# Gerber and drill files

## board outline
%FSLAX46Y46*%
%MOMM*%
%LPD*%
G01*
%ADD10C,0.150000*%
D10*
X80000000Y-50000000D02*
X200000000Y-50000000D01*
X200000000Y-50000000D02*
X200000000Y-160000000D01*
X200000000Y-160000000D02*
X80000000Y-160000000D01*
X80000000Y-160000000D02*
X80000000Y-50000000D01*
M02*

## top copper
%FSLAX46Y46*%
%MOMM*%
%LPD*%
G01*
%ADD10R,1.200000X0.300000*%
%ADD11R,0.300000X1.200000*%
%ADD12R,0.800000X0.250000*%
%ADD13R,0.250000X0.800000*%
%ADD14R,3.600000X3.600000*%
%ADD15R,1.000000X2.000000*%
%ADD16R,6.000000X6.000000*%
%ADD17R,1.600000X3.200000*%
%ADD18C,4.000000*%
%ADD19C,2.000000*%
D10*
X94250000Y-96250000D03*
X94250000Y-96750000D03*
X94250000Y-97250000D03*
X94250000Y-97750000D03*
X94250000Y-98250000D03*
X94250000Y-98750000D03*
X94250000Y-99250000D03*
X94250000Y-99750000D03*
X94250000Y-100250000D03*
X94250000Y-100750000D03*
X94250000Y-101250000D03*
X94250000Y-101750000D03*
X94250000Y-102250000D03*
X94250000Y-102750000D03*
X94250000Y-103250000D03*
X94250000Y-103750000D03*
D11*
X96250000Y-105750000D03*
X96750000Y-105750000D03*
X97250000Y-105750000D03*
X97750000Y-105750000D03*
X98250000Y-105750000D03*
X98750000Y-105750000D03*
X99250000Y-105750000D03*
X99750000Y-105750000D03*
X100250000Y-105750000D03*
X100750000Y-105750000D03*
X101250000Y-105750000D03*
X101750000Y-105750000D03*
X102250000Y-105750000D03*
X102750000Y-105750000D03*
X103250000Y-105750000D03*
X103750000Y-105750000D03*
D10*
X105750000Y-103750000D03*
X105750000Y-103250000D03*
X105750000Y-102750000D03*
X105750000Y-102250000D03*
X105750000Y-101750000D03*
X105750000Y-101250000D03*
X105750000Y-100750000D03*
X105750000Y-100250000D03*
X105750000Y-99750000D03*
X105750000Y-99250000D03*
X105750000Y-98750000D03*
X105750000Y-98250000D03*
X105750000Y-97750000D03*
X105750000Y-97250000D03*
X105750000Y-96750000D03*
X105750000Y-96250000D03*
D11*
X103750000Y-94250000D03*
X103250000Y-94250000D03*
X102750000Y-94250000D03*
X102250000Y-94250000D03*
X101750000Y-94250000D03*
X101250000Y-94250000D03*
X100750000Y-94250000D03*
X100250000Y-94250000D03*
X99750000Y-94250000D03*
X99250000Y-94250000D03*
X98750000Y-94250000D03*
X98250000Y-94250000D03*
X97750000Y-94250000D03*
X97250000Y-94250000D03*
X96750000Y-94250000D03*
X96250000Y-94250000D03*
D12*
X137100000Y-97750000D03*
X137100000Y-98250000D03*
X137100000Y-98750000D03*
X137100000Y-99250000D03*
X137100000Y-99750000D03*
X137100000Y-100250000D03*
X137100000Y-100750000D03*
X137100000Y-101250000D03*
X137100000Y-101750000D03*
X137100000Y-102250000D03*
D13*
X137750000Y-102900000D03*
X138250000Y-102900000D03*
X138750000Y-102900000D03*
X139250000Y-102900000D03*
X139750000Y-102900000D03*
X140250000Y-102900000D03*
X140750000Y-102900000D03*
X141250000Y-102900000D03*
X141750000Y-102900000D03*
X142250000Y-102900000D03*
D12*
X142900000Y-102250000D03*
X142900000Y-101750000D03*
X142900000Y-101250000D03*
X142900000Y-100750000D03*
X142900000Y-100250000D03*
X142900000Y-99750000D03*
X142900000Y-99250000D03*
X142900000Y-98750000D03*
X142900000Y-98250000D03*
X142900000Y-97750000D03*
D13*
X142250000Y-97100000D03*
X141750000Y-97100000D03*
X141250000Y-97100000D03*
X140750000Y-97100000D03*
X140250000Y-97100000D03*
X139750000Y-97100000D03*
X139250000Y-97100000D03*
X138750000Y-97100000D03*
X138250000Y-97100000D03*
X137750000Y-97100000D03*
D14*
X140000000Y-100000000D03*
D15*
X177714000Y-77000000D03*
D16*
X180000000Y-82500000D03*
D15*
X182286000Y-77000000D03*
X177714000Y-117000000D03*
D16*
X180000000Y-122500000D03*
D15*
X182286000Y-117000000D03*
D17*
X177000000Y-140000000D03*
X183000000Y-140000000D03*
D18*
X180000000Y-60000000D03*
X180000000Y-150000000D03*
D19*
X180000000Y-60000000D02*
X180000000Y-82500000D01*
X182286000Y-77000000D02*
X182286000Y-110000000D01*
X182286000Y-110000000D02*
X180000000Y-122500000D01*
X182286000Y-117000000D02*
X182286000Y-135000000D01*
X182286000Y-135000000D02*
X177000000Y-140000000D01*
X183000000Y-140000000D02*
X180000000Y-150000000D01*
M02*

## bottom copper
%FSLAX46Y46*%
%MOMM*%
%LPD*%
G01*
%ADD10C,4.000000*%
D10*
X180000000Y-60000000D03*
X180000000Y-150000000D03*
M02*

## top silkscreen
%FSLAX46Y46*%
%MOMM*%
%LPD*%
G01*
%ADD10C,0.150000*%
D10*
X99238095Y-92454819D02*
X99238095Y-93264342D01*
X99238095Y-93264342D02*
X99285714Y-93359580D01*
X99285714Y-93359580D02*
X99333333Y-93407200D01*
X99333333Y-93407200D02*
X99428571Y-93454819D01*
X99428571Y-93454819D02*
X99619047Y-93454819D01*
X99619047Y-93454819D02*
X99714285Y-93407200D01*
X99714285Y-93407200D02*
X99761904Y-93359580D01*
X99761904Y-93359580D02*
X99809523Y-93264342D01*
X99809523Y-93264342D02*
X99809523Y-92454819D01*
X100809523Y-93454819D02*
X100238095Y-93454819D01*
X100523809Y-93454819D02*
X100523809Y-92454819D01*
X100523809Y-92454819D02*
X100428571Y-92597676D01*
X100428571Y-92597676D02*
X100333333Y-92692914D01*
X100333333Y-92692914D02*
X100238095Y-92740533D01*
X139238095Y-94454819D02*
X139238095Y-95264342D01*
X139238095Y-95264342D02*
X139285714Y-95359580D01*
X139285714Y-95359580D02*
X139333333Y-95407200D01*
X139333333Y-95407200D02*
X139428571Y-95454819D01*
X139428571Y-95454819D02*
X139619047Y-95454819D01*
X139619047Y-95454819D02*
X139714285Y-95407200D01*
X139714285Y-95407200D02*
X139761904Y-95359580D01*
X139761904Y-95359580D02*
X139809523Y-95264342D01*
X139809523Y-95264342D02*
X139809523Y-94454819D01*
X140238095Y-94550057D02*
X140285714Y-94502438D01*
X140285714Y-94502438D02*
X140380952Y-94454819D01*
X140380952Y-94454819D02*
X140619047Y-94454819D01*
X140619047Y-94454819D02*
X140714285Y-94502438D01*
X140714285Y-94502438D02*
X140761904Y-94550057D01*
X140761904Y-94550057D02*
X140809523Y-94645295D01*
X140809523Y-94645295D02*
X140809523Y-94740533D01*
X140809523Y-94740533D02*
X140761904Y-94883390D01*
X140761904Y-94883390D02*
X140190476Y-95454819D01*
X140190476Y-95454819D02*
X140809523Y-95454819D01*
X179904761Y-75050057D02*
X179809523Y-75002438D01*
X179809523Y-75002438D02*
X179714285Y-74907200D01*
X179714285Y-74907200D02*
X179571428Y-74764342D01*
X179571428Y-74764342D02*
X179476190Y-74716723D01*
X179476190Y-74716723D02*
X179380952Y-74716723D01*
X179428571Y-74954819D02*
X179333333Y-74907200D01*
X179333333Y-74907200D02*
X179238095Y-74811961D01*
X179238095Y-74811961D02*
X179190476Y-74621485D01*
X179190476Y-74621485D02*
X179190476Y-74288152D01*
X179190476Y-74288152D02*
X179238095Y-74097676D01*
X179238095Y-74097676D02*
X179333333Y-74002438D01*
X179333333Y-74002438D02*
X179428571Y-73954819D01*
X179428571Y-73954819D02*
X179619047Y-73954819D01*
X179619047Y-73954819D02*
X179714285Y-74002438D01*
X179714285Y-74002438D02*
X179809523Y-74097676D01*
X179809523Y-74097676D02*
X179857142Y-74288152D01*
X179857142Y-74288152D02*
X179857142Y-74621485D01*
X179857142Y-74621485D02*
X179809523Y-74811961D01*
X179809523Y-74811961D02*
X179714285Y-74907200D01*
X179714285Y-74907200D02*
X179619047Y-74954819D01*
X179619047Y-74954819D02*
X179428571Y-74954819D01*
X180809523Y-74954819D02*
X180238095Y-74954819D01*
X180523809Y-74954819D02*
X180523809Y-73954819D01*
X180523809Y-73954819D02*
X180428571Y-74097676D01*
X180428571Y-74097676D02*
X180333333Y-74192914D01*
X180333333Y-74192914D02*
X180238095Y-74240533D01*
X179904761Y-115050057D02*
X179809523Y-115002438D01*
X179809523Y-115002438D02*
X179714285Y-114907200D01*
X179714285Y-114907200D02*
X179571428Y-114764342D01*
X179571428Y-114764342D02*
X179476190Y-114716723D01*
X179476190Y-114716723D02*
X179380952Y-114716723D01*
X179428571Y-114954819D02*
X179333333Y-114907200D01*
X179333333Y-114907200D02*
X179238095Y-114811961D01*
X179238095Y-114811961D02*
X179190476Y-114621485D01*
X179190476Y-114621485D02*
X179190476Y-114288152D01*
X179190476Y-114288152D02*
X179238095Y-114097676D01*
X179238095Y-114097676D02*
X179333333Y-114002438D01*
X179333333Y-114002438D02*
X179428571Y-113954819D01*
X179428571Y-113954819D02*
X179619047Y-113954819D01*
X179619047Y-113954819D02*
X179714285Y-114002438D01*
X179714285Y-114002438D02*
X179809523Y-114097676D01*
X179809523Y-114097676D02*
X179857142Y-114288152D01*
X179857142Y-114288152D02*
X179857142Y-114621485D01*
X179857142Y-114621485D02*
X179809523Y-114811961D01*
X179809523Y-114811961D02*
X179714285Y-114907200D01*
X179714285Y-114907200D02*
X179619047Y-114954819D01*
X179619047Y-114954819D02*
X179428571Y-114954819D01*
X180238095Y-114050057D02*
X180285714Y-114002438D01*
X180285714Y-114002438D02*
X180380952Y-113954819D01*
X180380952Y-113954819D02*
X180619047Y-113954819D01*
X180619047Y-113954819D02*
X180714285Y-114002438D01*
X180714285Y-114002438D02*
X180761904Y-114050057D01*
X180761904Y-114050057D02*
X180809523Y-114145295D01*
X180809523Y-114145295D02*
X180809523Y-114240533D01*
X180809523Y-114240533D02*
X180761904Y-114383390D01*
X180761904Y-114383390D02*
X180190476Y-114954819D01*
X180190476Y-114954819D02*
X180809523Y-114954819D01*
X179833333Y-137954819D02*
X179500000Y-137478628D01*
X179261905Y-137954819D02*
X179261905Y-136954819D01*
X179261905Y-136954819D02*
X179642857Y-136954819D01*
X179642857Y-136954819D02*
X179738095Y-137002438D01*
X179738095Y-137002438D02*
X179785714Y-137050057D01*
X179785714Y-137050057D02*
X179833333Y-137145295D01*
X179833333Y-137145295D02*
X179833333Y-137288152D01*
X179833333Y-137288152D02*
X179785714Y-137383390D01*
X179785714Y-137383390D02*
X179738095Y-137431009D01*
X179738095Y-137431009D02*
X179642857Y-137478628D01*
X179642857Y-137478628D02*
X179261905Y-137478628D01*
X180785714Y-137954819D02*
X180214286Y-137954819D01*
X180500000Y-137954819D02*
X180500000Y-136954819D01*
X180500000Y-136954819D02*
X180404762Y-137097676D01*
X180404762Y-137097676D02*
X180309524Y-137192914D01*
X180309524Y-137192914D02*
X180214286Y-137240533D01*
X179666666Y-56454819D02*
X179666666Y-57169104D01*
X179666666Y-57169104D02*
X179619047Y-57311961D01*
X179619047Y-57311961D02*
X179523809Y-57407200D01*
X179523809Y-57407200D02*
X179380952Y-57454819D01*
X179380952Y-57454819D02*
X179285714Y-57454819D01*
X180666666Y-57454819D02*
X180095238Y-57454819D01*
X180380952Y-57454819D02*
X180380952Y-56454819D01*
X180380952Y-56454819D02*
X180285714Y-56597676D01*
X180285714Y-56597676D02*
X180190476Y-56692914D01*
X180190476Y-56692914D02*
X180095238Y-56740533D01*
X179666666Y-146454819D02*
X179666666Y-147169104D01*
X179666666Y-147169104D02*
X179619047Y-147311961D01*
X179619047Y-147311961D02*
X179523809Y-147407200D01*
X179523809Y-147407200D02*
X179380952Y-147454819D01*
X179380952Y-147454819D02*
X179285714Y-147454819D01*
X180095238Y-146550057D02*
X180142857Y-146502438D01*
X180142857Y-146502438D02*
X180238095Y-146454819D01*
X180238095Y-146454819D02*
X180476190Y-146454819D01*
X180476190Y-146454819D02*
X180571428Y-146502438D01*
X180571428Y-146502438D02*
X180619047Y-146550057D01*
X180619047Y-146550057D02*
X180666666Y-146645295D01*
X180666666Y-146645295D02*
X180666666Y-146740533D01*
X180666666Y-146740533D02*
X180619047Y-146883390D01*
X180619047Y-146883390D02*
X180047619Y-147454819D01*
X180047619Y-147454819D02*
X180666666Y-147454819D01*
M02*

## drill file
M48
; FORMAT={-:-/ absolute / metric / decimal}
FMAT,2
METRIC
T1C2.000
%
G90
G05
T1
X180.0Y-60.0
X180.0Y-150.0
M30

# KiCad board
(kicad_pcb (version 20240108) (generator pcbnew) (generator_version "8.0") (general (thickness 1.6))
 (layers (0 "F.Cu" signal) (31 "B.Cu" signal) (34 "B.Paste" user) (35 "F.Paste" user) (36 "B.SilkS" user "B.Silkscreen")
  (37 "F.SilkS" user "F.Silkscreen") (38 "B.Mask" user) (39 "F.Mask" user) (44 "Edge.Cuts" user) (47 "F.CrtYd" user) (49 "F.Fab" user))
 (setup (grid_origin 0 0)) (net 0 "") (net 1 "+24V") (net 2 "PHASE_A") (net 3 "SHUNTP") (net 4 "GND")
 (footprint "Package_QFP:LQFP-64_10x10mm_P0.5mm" (layer "F.Cu") (at 100.0 100.0)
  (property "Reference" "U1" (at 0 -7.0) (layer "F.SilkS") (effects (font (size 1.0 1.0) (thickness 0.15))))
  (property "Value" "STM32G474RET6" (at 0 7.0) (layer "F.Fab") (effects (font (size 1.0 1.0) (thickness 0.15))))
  (pad "1" smd rect (at -5.75 -3.75) (size 1.2 0.3) (layers "F.Cu" "F.Paste" "F.Mask"))
  (pad "2" smd rect (at -5.75 -3.25) (size 1.2 0.3) (layers "F.Cu" "F.Paste" "F.Mask"))
  (pad "3" smd rect (at -5.75 -2.75) (size 1.2 0.3) (layers "F.Cu" "F.Paste" "F.Mask"))
  (pad "4" smd rect (at -5.75 -2.25) (size 1.2 0.3) (layers "F.Cu" "F.Paste" "F.Mask"))
  (pad "5" smd rect (at -5.75 -1.75) (size 1.2 0.3) (layers "F.Cu" "F.Paste" "F.Mask"))
  (pad "6" smd rect (at -5.75 -1.25) (size 1.2 0.3) (layers "F.Cu" "F.Paste" "F.Mask"))
  (pad "7" smd rect (at -5.75 -0.75) (size 1.2 0.3) (layers "F.Cu" "F.Paste" "F.Mask"))
  (pad "8" smd rect (at -5.75 -0.25) (size 1.2 0.3) (layers "F.Cu" "F.Paste" "F.Mask"))
  (pad "9" smd rect (at -5.75 0.25) (size 1.2 0.3) (layers "F.Cu" "F.Paste" "F.Mask"))
  (pad "10" smd rect (at -5.75 0.75) (size 1.2 0.3) (layers "F.Cu" "F.Paste" "F.Mask"))
  (pad "11" smd rect (at -5.75 1.25) (size 1.2 0.3) (layers "F.Cu" "F.Paste" "F.Mask"))
  (pad "12" smd rect (at -5.75 1.75) (size 1.2 0.3) (layers "F.Cu" "F.Paste" "F.Mask"))
  (pad "13" smd rect (at -5.75 2.25) (size 1.2 0.3) (layers "F.Cu" "F.Paste" "F.Mask"))
  (pad "14" smd rect (at -5.75 2.75) (size 1.2 0.3) (layers "F.Cu" "F.Paste" "F.Mask"))
  (pad "15" smd rect (at -5.75 3.25) (size 1.2 0.3) (layers "F.Cu" "F.Paste" "F.Mask"))
  (pad "16" smd rect (at -5.75 3.75) (size 1.2 0.3) (layers "F.Cu" "F.Paste" "F.Mask"))
  (pad "17" smd rect (at -3.75 5.75 90) (size 1.2 0.3) (layers "F.Cu" "F.Paste" "F.Mask"))
  (pad "18" smd rect (at -3.25 5.75 90) (size 1.2 0.3) (layers "F.Cu" "F.Paste" "F.Mask"))
  (pad "19" smd rect (at -2.75 5.75 90) (size 1.2 0.3) (layers "F.Cu" "F.Paste" "F.Mask"))
  (pad "20" smd rect (at -2.25 5.75 90) (size 1.2 0.3) (layers "F.Cu" "F.Paste" "F.Mask"))
  (pad "21" smd rect (at -1.75 5.75 90) (size 1.2 0.3) (layers "F.Cu" "F.Paste" "F.Mask"))
  (pad "22" smd rect (at -1.25 5.75 90) (size 1.2 0.3) (layers "F.Cu" "F.Paste" "F.Mask"))
  (pad "23" smd rect (at -0.75 5.75 90) (size 1.2 0.3) (layers "F.Cu" "F.Paste" "F.Mask"))
  (pad "24" smd rect (at -0.25 5.75 90) (size 1.2 0.3) (layers "F.Cu" "F.Paste" "F.Mask"))
  (pad "25" smd rect (at 0.25 5.75 90) (size 1.2 0.3) (layers "F.Cu" "F.Paste" "F.Mask"))
  (pad "26" smd rect (at 0.75 5.75 90) (size 1.2 0.3) (layers "F.Cu" "F.Paste" "F.Mask"))
  (pad "27" smd rect (at 1.25 5.75 90) (size 1.2 0.3) (layers "F.Cu" "F.Paste" "F.Mask"))
  (pad "28" smd rect (at 1.75 5.75 90) (size 1.2 0.3) (layers "F.Cu" "F.Paste" "F.Mask"))
  (pad "29" smd rect (at 2.25 5.75 90) (size 1.2 0.3) (layers "F.Cu" "F.Paste" "F.Mask"))
  (pad "30" smd rect (at 2.75 5.75 90) (size 1.2 0.3) (layers "F.Cu" "F.Paste" "F.Mask"))
  (pad "31" smd rect (at 3.25 5.75 90) (size 1.2 0.3) (layers "F.Cu" "F.Paste" "F.Mask"))
  (pad "32" smd rect (at 3.75 5.75 90) (size 1.2 0.3) (layers "F.Cu" "F.Paste" "F.Mask"))
  (pad "33" smd rect (at 5.75 3.75) (size 1.2 0.3) (layers "F.Cu" "F.Paste" "F.Mask"))
  (pad "34" smd rect (at 5.75 3.25) (size 1.2 0.3) (layers "F.Cu" "F.Paste" "F.Mask"))
  (pad "35" smd rect (at 5.75 2.75) (size 1.2 0.3) (layers "F.Cu" "F.Paste" "F.Mask"))
  (pad "36" smd rect (at 5.75 2.25) (size 1.2 0.3) (layers "F.Cu" "F.Paste" "F.Mask"))
  (pad "37" smd rect (at 5.75 1.75) (size 1.2 0.3) (layers "F.Cu" "F.Paste" "F.Mask"))
  (pad "38" smd rect (at 5.75 1.25) (size 1.2 0.3) (layers "F.Cu" "F.Paste" "F.Mask"))
  (pad "39" smd rect (at 5.75 0.75) (size 1.2 0.3) (layers "F.Cu" "F.Paste" "F.Mask"))
  (pad "40" smd rect (at 5.75 0.25) (size 1.2 0.3) (layers "F.Cu" "F.Paste" "F.Mask"))
  (pad "41" smd rect (at 5.75 -0.25) (size 1.2 0.3) (layers "F.Cu" "F.Paste" "F.Mask"))
  (pad "42" smd rect (at 5.75 -0.75) (size 1.2 0.3) (layers "F.Cu" "F.Paste" "F.Mask"))
  (pad "43" smd rect (at 5.75 -1.25) (size 1.2 0.3) (layers "F.Cu" "F.Paste" "F.Mask"))
  (pad "44" smd rect (at 5.75 -1.75) (size 1.2 0.3) (layers "F.Cu" "F.Paste" "F.Mask"))
  (pad "45" smd rect (at 5.75 -2.25) (size 1.2 0.3) (layers "F.Cu" "F.Paste" "F.Mask"))
  (pad "46" smd rect (at 5.75 -2.75) (size 1.2 0.3) (layers "F.Cu" "F.Paste" "F.Mask"))
  (pad "47" smd rect (at 5.75 -3.25) (size 1.2 0.3) (layers "F.Cu" "F.Paste" "F.Mask"))
  (pad "48" smd rect (at 5.75 -3.75) (size 1.2 0.3) (layers "F.Cu" "F.Paste" "F.Mask"))
  (pad "49" smd rect (at 3.75 -5.75 90) (size 1.2 0.3) (layers "F.Cu" "F.Paste" "F.Mask"))
  (pad "50" smd rect (at 3.25 -5.75 90) (size 1.2 0.3) (layers "F.Cu" "F.Paste" "F.Mask"))
  (pad "51" smd rect (at 2.75 -5.75 90) (size 1.2 0.3) (layers "F.Cu" "F.Paste" "F.Mask"))
  (pad "52" smd rect (at 2.25 -5.75 90) (size 1.2 0.3) (layers "F.Cu" "F.Paste" "F.Mask"))
  (pad "53" smd rect (at 1.75 -5.75 90) (size 1.2 0.3) (layers "F.Cu" "F.Paste" "F.Mask"))
  (pad "54" smd rect (at 1.25 -5.75 90) (size 1.2 0.3) (layers "F.Cu" "F.Paste" "F.Mask"))
  (pad "55" smd rect (at 0.75 -5.75 90) (size 1.2 0.3) (layers "F.Cu" "F.Paste" "F.Mask"))
  (pad "56" smd rect (at 0.25 -5.75 90) (size 1.2 0.3) (layers "F.Cu" "F.Paste" "F.Mask"))
  (pad "57" smd rect (at -0.25 -5.75 90) (size 1.2 0.3) (layers "F.Cu" "F.Paste" "F.Mask"))
  (pad "58" smd rect (at -0.75 -5.75 90) (size 1.2 0.3) (layers "F.Cu" "F.Paste" "F.Mask"))
  (pad "59" smd rect (at -1.25 -5.75 90) (size 1.2 0.3) (layers "F.Cu" "F.Paste" "F.Mask"))
  (pad "60" smd rect (at -1.75 -5.75 90) (size 1.2 0.3) (layers "F.Cu" "F.Paste" "F.Mask"))
  (pad "61" smd rect (at -2.25 -5.75 90) (size 1.2 0.3) (layers "F.Cu" "F.Paste" "F.Mask"))
  (pad "62" smd rect (at -2.75 -5.75 90) (size 1.2 0.3) (layers "F.Cu" "F.Paste" "F.Mask"))
  (pad "63" smd rect (at -3.25 -5.75 90) (size 1.2 0.3) (layers "F.Cu" "F.Paste" "F.Mask"))
  (pad "64" smd rect (at -3.75 -5.75 90) (size 1.2 0.3) (layers "F.Cu" "F.Paste" "F.Mask")))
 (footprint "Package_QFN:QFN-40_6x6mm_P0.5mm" (layer "F.Cu") (at 140.0 100.0)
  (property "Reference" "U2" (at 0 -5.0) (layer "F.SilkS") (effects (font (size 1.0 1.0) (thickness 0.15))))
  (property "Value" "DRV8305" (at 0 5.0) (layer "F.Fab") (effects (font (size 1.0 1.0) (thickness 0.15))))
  (pad "1" smd rect (at -2.9 -2.25) (size 0.8 0.25) (layers "F.Cu" "F.Paste" "F.Mask"))
  (pad "2" smd rect (at -2.9 -1.75) (size 0.8 0.25) (layers "F.Cu" "F.Paste" "F.Mask"))
  (pad "3" smd rect (at -2.9 -1.25) (size 0.8 0.25) (layers "F.Cu" "F.Paste" "F.Mask"))
  (pad "4" smd rect (at -2.9 -0.75) (size 0.8 0.25) (layers "F.Cu" "F.Paste" "F.Mask"))
  (pad "5" smd rect (at -2.9 -0.25) (size 0.8 0.25) (layers "F.Cu" "F.Paste" "F.Mask"))
  (pad "6" smd rect (at -2.9 0.25) (size 0.8 0.25) (layers "F.Cu" "F.Paste" "F.Mask"))
  (pad "7" smd rect (at -2.9 0.75) (size 0.8 0.25) (layers "F.Cu" "F.Paste" "F.Mask"))
  (pad "8" smd rect (at -2.9 1.25) (size 0.8 0.25) (layers "F.Cu" "F.Paste" "F.Mask"))
  (pad "9" smd rect (at -2.9 1.75) (size 0.8 0.25) (layers "F.Cu" "F.Paste" "F.Mask"))
  (pad "10" smd rect (at -2.9 2.25) (size 0.8 0.25) (layers "F.Cu" "F.Paste" "F.Mask"))
  (pad "11" smd rect (at -2.25 2.9 90) (size 0.8 0.25) (layers "F.Cu" "F.Paste" "F.Mask"))
  (pad "12" smd rect (at -1.75 2.9 90) (size 0.8 0.25) (layers "F.Cu" "F.Paste" "F.Mask"))
  (pad "13" smd rect (at -1.25 2.9 90) (size 0.8 0.25) (layers "F.Cu" "F.Paste" "F.Mask"))
  (pad "14" smd rect (at -0.75 2.9 90) (size 0.8 0.25) (layers "F.Cu" "F.Paste" "F.Mask"))
  (pad "15" smd rect (at -0.25 2.9 90) (size 0.8 0.25) (layers "F.Cu" "F.Paste" "F.Mask"))
  (pad "16" smd rect (at 0.25 2.9 90) (size 0.8 0.25) (layers "F.Cu" "F.Paste" "F.Mask"))
  (pad "17" smd rect (at 0.75 2.9 90) (size 0.8 0.25) (layers "F.Cu" "F.Paste" "F.Mask"))
  (pad "18" smd rect (at 1.25 2.9 90) (size 0.8 0.25) (layers "F.Cu" "F.Paste" "F.Mask"))
  (pad "19" smd rect (at 1.75 2.9 90) (size 0.8 0.25) (layers "F.Cu" "F.Paste" "F.Mask"))
  (pad "20" smd rect (at 2.25 2.9 90) (size 0.8 0.25) (layers "F.Cu" "F.Paste" "F.Mask"))
  (pad "21" smd rect (at 2.9 2.25) (size 0.8 0.25) (layers "F.Cu" "F.Paste" "F.Mask"))
  (pad "22" smd rect (at 2.9 1.75) (size 0.8 0.25) (layers "F.Cu" "F.Paste" "F.Mask"))
  (pad "23" smd rect (at 2.9 1.25) (size 0.8 0.25) (layers "F.Cu" "F.Paste" "F.Mask"))
  (pad "24" smd rect (at 2.9 0.75) (size 0.8 0.25) (layers "F.Cu" "F.Paste" "F.Mask"))
  (pad "25" smd rect (at 2.9 0.25) (size 0.8 0.25) (layers "F.Cu" "F.Paste" "F.Mask"))
  (pad "26" smd rect (at 2.9 -0.25) (size 0.8 0.25) (layers "F.Cu" "F.Paste" "F.Mask"))
  (pad "27" smd rect (at 2.9 -0.75) (size 0.8 0.25) (layers "F.Cu" "F.Paste" "F.Mask"))
  (pad "28" smd rect (at 2.9 -1.25) (size 0.8 0.25) (layers "F.Cu" "F.Paste" "F.Mask"))
  (pad "29" smd rect (at 2.9 -1.75) (size 0.8 0.25) (layers "F.Cu" "F.Paste" "F.Mask"))
  (pad "30" smd rect (at 2.9 -2.25) (size 0.8 0.25) (layers "F.Cu" "F.Paste" "F.Mask"))
  (pad "31" smd rect (at 2.25 -2.9 90) (size 0.8 0.25) (layers "F.Cu" "F.Paste" "F.Mask"))
  (pad "32" smd rect (at 1.75 -2.9 90) (size 0.8 0.25) (layers "F.Cu" "F.Paste" "F.Mask"))
  (pad "33" smd rect (at 1.25 -2.9 90) (size 0.8 0.25) (layers "F.Cu" "F.Paste" "F.Mask"))
  (pad "34" smd rect (at 0.75 -2.9 90) (size 0.8 0.25) (layers "F.Cu" "F.Paste" "F.Mask"))
  (pad "35" smd rect (at 0.25 -2.9 90) (size 0.8 0.25) (layers "F.Cu" "F.Paste" "F.Mask"))
  (pad "36" smd rect (at -0.25 -2.9 90) (size 0.8 0.25) (layers "F.Cu" "F.Paste" "F.Mask"))
  (pad "37" smd rect (at -0.75 -2.9 90) (size 0.8 0.25) (layers "F.Cu" "F.Paste" "F.Mask"))
  (pad "38" smd rect (at -1.25 -2.9 90) (size 0.8 0.25) (layers "F.Cu" "F.Paste" "F.Mask"))
  (pad "39" smd rect (at -1.75 -2.9 90) (size 0.8 0.25) (layers "F.Cu" "F.Paste" "F.Mask"))
  (pad "40" smd rect (at -2.25 -2.9 90) (size 0.8 0.25) (layers "F.Cu" "F.Paste" "F.Mask"))
  (pad "41" smd rect (at 0 0) (size 3.6 3.6) (layers "F.Cu" "F.Paste" "F.Mask")))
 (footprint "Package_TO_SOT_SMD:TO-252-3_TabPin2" (layer "F.Cu") (at 180.0 80.0)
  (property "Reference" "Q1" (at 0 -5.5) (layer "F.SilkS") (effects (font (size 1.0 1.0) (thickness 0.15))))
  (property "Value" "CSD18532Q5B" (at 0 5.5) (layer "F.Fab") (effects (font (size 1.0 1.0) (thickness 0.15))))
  (pad "1" smd rect (at -2.286 -3.0) (size 1.0 2.0) (layers "F.Cu" "F.Paste" "F.Mask"))
  (pad "2" smd rect (at 0.0 2.5) (size 6.0 6.0) (layers "F.Cu" "F.Paste" "F.Mask") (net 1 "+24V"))
  (pad "3" smd rect (at 2.286 -3.0) (size 1.0 2.0) (layers "F.Cu" "F.Paste" "F.Mask") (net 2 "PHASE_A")))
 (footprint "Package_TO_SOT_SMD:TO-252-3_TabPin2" (layer "F.Cu") (at 180.0 120.0)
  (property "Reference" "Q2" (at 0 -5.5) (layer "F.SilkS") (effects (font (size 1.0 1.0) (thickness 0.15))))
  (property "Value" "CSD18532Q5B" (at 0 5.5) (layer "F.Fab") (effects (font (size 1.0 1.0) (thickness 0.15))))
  (pad "1" smd rect (at -2.286 -3.0) (size 1.0 2.0) (layers "F.Cu" "F.Paste" "F.Mask"))
  (pad "2" smd rect (at 0.0 2.5) (size 6.0 6.0) (layers "F.Cu" "F.Paste" "F.Mask") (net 2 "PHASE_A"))
  (pad "3" smd rect (at 2.286 -3.0) (size 1.0 2.0) (layers "F.Cu" "F.Paste" "F.Mask") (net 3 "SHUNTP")))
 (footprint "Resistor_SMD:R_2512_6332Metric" (layer "F.Cu") (at 180.0 140.0)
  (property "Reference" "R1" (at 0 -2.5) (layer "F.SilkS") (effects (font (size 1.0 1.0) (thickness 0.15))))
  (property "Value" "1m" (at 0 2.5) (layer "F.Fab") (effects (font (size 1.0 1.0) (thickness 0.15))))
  (pad "1" smd rect (at -3.0 0.0) (size 1.6 3.2) (layers "F.Cu" "F.Paste" "F.Mask") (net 3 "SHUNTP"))
  (pad "2" smd rect (at 3.0 0.0) (size 1.6 3.2) (layers "F.Cu" "F.Paste" "F.Mask") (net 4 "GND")))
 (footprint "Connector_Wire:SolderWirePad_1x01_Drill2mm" (layer "F.Cu") (at 180.0 60.0)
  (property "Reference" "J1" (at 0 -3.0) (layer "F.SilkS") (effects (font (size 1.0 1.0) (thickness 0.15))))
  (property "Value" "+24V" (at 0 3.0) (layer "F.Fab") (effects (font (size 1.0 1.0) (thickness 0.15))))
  (pad "1" thru_hole circle (at 0 0) (size 4.0 4.0) (drill 2.0) (layers "*.Cu" "*.Mask") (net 1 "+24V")))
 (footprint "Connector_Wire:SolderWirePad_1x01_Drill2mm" (layer "F.Cu") (at 180.0 150.0)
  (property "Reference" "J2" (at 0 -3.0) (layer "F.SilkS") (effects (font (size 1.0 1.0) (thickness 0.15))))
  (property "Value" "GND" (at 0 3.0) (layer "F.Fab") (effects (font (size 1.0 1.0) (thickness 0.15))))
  (pad "1" thru_hole circle (at 0 0) (size 4.0 4.0) (drill 2.0) (layers "*.Cu" "*.Mask") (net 4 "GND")))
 (gr_line (start 80.0 50.0) (end 200.0 50.0) (layer "Edge.Cuts") (width 0.15))
 (gr_line (start 200.0 50.0) (end 200.0 160.0) (layer "Edge.Cuts") (width 0.15))
 (gr_line (start 200.0 160.0) (end 80.0 160.0) (layer "Edge.Cuts") (width 0.15))
 (gr_line (start 80.0 160.0) (end 80.0 50.0) (layer "Edge.Cuts") (width 0.15))
 (segment (start 180.0 60.0) (end 180.0 82.5) (width 2.0) (layer "F.Cu") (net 1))
 (segment (start 182.286 77.0) (end 182.286 110.0) (width 2.0) (layer "F.Cu") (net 2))
 (segment (start 182.286 110.0) (end 180.0 122.5) (width 2.0) (layer "F.Cu") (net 2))
 (segment (start 182.286 117.0) (end 182.286 135.0) (width 2.0) (layer "F.Cu") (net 3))
 (segment (start 182.286 135.0) (end 177.0 140.0) (width 2.0) (layer "F.Cu") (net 3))
 (segment (start 183.0 140.0) (end 180.0 150.0) (width 2.0) (layer "F.Cu") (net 4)))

